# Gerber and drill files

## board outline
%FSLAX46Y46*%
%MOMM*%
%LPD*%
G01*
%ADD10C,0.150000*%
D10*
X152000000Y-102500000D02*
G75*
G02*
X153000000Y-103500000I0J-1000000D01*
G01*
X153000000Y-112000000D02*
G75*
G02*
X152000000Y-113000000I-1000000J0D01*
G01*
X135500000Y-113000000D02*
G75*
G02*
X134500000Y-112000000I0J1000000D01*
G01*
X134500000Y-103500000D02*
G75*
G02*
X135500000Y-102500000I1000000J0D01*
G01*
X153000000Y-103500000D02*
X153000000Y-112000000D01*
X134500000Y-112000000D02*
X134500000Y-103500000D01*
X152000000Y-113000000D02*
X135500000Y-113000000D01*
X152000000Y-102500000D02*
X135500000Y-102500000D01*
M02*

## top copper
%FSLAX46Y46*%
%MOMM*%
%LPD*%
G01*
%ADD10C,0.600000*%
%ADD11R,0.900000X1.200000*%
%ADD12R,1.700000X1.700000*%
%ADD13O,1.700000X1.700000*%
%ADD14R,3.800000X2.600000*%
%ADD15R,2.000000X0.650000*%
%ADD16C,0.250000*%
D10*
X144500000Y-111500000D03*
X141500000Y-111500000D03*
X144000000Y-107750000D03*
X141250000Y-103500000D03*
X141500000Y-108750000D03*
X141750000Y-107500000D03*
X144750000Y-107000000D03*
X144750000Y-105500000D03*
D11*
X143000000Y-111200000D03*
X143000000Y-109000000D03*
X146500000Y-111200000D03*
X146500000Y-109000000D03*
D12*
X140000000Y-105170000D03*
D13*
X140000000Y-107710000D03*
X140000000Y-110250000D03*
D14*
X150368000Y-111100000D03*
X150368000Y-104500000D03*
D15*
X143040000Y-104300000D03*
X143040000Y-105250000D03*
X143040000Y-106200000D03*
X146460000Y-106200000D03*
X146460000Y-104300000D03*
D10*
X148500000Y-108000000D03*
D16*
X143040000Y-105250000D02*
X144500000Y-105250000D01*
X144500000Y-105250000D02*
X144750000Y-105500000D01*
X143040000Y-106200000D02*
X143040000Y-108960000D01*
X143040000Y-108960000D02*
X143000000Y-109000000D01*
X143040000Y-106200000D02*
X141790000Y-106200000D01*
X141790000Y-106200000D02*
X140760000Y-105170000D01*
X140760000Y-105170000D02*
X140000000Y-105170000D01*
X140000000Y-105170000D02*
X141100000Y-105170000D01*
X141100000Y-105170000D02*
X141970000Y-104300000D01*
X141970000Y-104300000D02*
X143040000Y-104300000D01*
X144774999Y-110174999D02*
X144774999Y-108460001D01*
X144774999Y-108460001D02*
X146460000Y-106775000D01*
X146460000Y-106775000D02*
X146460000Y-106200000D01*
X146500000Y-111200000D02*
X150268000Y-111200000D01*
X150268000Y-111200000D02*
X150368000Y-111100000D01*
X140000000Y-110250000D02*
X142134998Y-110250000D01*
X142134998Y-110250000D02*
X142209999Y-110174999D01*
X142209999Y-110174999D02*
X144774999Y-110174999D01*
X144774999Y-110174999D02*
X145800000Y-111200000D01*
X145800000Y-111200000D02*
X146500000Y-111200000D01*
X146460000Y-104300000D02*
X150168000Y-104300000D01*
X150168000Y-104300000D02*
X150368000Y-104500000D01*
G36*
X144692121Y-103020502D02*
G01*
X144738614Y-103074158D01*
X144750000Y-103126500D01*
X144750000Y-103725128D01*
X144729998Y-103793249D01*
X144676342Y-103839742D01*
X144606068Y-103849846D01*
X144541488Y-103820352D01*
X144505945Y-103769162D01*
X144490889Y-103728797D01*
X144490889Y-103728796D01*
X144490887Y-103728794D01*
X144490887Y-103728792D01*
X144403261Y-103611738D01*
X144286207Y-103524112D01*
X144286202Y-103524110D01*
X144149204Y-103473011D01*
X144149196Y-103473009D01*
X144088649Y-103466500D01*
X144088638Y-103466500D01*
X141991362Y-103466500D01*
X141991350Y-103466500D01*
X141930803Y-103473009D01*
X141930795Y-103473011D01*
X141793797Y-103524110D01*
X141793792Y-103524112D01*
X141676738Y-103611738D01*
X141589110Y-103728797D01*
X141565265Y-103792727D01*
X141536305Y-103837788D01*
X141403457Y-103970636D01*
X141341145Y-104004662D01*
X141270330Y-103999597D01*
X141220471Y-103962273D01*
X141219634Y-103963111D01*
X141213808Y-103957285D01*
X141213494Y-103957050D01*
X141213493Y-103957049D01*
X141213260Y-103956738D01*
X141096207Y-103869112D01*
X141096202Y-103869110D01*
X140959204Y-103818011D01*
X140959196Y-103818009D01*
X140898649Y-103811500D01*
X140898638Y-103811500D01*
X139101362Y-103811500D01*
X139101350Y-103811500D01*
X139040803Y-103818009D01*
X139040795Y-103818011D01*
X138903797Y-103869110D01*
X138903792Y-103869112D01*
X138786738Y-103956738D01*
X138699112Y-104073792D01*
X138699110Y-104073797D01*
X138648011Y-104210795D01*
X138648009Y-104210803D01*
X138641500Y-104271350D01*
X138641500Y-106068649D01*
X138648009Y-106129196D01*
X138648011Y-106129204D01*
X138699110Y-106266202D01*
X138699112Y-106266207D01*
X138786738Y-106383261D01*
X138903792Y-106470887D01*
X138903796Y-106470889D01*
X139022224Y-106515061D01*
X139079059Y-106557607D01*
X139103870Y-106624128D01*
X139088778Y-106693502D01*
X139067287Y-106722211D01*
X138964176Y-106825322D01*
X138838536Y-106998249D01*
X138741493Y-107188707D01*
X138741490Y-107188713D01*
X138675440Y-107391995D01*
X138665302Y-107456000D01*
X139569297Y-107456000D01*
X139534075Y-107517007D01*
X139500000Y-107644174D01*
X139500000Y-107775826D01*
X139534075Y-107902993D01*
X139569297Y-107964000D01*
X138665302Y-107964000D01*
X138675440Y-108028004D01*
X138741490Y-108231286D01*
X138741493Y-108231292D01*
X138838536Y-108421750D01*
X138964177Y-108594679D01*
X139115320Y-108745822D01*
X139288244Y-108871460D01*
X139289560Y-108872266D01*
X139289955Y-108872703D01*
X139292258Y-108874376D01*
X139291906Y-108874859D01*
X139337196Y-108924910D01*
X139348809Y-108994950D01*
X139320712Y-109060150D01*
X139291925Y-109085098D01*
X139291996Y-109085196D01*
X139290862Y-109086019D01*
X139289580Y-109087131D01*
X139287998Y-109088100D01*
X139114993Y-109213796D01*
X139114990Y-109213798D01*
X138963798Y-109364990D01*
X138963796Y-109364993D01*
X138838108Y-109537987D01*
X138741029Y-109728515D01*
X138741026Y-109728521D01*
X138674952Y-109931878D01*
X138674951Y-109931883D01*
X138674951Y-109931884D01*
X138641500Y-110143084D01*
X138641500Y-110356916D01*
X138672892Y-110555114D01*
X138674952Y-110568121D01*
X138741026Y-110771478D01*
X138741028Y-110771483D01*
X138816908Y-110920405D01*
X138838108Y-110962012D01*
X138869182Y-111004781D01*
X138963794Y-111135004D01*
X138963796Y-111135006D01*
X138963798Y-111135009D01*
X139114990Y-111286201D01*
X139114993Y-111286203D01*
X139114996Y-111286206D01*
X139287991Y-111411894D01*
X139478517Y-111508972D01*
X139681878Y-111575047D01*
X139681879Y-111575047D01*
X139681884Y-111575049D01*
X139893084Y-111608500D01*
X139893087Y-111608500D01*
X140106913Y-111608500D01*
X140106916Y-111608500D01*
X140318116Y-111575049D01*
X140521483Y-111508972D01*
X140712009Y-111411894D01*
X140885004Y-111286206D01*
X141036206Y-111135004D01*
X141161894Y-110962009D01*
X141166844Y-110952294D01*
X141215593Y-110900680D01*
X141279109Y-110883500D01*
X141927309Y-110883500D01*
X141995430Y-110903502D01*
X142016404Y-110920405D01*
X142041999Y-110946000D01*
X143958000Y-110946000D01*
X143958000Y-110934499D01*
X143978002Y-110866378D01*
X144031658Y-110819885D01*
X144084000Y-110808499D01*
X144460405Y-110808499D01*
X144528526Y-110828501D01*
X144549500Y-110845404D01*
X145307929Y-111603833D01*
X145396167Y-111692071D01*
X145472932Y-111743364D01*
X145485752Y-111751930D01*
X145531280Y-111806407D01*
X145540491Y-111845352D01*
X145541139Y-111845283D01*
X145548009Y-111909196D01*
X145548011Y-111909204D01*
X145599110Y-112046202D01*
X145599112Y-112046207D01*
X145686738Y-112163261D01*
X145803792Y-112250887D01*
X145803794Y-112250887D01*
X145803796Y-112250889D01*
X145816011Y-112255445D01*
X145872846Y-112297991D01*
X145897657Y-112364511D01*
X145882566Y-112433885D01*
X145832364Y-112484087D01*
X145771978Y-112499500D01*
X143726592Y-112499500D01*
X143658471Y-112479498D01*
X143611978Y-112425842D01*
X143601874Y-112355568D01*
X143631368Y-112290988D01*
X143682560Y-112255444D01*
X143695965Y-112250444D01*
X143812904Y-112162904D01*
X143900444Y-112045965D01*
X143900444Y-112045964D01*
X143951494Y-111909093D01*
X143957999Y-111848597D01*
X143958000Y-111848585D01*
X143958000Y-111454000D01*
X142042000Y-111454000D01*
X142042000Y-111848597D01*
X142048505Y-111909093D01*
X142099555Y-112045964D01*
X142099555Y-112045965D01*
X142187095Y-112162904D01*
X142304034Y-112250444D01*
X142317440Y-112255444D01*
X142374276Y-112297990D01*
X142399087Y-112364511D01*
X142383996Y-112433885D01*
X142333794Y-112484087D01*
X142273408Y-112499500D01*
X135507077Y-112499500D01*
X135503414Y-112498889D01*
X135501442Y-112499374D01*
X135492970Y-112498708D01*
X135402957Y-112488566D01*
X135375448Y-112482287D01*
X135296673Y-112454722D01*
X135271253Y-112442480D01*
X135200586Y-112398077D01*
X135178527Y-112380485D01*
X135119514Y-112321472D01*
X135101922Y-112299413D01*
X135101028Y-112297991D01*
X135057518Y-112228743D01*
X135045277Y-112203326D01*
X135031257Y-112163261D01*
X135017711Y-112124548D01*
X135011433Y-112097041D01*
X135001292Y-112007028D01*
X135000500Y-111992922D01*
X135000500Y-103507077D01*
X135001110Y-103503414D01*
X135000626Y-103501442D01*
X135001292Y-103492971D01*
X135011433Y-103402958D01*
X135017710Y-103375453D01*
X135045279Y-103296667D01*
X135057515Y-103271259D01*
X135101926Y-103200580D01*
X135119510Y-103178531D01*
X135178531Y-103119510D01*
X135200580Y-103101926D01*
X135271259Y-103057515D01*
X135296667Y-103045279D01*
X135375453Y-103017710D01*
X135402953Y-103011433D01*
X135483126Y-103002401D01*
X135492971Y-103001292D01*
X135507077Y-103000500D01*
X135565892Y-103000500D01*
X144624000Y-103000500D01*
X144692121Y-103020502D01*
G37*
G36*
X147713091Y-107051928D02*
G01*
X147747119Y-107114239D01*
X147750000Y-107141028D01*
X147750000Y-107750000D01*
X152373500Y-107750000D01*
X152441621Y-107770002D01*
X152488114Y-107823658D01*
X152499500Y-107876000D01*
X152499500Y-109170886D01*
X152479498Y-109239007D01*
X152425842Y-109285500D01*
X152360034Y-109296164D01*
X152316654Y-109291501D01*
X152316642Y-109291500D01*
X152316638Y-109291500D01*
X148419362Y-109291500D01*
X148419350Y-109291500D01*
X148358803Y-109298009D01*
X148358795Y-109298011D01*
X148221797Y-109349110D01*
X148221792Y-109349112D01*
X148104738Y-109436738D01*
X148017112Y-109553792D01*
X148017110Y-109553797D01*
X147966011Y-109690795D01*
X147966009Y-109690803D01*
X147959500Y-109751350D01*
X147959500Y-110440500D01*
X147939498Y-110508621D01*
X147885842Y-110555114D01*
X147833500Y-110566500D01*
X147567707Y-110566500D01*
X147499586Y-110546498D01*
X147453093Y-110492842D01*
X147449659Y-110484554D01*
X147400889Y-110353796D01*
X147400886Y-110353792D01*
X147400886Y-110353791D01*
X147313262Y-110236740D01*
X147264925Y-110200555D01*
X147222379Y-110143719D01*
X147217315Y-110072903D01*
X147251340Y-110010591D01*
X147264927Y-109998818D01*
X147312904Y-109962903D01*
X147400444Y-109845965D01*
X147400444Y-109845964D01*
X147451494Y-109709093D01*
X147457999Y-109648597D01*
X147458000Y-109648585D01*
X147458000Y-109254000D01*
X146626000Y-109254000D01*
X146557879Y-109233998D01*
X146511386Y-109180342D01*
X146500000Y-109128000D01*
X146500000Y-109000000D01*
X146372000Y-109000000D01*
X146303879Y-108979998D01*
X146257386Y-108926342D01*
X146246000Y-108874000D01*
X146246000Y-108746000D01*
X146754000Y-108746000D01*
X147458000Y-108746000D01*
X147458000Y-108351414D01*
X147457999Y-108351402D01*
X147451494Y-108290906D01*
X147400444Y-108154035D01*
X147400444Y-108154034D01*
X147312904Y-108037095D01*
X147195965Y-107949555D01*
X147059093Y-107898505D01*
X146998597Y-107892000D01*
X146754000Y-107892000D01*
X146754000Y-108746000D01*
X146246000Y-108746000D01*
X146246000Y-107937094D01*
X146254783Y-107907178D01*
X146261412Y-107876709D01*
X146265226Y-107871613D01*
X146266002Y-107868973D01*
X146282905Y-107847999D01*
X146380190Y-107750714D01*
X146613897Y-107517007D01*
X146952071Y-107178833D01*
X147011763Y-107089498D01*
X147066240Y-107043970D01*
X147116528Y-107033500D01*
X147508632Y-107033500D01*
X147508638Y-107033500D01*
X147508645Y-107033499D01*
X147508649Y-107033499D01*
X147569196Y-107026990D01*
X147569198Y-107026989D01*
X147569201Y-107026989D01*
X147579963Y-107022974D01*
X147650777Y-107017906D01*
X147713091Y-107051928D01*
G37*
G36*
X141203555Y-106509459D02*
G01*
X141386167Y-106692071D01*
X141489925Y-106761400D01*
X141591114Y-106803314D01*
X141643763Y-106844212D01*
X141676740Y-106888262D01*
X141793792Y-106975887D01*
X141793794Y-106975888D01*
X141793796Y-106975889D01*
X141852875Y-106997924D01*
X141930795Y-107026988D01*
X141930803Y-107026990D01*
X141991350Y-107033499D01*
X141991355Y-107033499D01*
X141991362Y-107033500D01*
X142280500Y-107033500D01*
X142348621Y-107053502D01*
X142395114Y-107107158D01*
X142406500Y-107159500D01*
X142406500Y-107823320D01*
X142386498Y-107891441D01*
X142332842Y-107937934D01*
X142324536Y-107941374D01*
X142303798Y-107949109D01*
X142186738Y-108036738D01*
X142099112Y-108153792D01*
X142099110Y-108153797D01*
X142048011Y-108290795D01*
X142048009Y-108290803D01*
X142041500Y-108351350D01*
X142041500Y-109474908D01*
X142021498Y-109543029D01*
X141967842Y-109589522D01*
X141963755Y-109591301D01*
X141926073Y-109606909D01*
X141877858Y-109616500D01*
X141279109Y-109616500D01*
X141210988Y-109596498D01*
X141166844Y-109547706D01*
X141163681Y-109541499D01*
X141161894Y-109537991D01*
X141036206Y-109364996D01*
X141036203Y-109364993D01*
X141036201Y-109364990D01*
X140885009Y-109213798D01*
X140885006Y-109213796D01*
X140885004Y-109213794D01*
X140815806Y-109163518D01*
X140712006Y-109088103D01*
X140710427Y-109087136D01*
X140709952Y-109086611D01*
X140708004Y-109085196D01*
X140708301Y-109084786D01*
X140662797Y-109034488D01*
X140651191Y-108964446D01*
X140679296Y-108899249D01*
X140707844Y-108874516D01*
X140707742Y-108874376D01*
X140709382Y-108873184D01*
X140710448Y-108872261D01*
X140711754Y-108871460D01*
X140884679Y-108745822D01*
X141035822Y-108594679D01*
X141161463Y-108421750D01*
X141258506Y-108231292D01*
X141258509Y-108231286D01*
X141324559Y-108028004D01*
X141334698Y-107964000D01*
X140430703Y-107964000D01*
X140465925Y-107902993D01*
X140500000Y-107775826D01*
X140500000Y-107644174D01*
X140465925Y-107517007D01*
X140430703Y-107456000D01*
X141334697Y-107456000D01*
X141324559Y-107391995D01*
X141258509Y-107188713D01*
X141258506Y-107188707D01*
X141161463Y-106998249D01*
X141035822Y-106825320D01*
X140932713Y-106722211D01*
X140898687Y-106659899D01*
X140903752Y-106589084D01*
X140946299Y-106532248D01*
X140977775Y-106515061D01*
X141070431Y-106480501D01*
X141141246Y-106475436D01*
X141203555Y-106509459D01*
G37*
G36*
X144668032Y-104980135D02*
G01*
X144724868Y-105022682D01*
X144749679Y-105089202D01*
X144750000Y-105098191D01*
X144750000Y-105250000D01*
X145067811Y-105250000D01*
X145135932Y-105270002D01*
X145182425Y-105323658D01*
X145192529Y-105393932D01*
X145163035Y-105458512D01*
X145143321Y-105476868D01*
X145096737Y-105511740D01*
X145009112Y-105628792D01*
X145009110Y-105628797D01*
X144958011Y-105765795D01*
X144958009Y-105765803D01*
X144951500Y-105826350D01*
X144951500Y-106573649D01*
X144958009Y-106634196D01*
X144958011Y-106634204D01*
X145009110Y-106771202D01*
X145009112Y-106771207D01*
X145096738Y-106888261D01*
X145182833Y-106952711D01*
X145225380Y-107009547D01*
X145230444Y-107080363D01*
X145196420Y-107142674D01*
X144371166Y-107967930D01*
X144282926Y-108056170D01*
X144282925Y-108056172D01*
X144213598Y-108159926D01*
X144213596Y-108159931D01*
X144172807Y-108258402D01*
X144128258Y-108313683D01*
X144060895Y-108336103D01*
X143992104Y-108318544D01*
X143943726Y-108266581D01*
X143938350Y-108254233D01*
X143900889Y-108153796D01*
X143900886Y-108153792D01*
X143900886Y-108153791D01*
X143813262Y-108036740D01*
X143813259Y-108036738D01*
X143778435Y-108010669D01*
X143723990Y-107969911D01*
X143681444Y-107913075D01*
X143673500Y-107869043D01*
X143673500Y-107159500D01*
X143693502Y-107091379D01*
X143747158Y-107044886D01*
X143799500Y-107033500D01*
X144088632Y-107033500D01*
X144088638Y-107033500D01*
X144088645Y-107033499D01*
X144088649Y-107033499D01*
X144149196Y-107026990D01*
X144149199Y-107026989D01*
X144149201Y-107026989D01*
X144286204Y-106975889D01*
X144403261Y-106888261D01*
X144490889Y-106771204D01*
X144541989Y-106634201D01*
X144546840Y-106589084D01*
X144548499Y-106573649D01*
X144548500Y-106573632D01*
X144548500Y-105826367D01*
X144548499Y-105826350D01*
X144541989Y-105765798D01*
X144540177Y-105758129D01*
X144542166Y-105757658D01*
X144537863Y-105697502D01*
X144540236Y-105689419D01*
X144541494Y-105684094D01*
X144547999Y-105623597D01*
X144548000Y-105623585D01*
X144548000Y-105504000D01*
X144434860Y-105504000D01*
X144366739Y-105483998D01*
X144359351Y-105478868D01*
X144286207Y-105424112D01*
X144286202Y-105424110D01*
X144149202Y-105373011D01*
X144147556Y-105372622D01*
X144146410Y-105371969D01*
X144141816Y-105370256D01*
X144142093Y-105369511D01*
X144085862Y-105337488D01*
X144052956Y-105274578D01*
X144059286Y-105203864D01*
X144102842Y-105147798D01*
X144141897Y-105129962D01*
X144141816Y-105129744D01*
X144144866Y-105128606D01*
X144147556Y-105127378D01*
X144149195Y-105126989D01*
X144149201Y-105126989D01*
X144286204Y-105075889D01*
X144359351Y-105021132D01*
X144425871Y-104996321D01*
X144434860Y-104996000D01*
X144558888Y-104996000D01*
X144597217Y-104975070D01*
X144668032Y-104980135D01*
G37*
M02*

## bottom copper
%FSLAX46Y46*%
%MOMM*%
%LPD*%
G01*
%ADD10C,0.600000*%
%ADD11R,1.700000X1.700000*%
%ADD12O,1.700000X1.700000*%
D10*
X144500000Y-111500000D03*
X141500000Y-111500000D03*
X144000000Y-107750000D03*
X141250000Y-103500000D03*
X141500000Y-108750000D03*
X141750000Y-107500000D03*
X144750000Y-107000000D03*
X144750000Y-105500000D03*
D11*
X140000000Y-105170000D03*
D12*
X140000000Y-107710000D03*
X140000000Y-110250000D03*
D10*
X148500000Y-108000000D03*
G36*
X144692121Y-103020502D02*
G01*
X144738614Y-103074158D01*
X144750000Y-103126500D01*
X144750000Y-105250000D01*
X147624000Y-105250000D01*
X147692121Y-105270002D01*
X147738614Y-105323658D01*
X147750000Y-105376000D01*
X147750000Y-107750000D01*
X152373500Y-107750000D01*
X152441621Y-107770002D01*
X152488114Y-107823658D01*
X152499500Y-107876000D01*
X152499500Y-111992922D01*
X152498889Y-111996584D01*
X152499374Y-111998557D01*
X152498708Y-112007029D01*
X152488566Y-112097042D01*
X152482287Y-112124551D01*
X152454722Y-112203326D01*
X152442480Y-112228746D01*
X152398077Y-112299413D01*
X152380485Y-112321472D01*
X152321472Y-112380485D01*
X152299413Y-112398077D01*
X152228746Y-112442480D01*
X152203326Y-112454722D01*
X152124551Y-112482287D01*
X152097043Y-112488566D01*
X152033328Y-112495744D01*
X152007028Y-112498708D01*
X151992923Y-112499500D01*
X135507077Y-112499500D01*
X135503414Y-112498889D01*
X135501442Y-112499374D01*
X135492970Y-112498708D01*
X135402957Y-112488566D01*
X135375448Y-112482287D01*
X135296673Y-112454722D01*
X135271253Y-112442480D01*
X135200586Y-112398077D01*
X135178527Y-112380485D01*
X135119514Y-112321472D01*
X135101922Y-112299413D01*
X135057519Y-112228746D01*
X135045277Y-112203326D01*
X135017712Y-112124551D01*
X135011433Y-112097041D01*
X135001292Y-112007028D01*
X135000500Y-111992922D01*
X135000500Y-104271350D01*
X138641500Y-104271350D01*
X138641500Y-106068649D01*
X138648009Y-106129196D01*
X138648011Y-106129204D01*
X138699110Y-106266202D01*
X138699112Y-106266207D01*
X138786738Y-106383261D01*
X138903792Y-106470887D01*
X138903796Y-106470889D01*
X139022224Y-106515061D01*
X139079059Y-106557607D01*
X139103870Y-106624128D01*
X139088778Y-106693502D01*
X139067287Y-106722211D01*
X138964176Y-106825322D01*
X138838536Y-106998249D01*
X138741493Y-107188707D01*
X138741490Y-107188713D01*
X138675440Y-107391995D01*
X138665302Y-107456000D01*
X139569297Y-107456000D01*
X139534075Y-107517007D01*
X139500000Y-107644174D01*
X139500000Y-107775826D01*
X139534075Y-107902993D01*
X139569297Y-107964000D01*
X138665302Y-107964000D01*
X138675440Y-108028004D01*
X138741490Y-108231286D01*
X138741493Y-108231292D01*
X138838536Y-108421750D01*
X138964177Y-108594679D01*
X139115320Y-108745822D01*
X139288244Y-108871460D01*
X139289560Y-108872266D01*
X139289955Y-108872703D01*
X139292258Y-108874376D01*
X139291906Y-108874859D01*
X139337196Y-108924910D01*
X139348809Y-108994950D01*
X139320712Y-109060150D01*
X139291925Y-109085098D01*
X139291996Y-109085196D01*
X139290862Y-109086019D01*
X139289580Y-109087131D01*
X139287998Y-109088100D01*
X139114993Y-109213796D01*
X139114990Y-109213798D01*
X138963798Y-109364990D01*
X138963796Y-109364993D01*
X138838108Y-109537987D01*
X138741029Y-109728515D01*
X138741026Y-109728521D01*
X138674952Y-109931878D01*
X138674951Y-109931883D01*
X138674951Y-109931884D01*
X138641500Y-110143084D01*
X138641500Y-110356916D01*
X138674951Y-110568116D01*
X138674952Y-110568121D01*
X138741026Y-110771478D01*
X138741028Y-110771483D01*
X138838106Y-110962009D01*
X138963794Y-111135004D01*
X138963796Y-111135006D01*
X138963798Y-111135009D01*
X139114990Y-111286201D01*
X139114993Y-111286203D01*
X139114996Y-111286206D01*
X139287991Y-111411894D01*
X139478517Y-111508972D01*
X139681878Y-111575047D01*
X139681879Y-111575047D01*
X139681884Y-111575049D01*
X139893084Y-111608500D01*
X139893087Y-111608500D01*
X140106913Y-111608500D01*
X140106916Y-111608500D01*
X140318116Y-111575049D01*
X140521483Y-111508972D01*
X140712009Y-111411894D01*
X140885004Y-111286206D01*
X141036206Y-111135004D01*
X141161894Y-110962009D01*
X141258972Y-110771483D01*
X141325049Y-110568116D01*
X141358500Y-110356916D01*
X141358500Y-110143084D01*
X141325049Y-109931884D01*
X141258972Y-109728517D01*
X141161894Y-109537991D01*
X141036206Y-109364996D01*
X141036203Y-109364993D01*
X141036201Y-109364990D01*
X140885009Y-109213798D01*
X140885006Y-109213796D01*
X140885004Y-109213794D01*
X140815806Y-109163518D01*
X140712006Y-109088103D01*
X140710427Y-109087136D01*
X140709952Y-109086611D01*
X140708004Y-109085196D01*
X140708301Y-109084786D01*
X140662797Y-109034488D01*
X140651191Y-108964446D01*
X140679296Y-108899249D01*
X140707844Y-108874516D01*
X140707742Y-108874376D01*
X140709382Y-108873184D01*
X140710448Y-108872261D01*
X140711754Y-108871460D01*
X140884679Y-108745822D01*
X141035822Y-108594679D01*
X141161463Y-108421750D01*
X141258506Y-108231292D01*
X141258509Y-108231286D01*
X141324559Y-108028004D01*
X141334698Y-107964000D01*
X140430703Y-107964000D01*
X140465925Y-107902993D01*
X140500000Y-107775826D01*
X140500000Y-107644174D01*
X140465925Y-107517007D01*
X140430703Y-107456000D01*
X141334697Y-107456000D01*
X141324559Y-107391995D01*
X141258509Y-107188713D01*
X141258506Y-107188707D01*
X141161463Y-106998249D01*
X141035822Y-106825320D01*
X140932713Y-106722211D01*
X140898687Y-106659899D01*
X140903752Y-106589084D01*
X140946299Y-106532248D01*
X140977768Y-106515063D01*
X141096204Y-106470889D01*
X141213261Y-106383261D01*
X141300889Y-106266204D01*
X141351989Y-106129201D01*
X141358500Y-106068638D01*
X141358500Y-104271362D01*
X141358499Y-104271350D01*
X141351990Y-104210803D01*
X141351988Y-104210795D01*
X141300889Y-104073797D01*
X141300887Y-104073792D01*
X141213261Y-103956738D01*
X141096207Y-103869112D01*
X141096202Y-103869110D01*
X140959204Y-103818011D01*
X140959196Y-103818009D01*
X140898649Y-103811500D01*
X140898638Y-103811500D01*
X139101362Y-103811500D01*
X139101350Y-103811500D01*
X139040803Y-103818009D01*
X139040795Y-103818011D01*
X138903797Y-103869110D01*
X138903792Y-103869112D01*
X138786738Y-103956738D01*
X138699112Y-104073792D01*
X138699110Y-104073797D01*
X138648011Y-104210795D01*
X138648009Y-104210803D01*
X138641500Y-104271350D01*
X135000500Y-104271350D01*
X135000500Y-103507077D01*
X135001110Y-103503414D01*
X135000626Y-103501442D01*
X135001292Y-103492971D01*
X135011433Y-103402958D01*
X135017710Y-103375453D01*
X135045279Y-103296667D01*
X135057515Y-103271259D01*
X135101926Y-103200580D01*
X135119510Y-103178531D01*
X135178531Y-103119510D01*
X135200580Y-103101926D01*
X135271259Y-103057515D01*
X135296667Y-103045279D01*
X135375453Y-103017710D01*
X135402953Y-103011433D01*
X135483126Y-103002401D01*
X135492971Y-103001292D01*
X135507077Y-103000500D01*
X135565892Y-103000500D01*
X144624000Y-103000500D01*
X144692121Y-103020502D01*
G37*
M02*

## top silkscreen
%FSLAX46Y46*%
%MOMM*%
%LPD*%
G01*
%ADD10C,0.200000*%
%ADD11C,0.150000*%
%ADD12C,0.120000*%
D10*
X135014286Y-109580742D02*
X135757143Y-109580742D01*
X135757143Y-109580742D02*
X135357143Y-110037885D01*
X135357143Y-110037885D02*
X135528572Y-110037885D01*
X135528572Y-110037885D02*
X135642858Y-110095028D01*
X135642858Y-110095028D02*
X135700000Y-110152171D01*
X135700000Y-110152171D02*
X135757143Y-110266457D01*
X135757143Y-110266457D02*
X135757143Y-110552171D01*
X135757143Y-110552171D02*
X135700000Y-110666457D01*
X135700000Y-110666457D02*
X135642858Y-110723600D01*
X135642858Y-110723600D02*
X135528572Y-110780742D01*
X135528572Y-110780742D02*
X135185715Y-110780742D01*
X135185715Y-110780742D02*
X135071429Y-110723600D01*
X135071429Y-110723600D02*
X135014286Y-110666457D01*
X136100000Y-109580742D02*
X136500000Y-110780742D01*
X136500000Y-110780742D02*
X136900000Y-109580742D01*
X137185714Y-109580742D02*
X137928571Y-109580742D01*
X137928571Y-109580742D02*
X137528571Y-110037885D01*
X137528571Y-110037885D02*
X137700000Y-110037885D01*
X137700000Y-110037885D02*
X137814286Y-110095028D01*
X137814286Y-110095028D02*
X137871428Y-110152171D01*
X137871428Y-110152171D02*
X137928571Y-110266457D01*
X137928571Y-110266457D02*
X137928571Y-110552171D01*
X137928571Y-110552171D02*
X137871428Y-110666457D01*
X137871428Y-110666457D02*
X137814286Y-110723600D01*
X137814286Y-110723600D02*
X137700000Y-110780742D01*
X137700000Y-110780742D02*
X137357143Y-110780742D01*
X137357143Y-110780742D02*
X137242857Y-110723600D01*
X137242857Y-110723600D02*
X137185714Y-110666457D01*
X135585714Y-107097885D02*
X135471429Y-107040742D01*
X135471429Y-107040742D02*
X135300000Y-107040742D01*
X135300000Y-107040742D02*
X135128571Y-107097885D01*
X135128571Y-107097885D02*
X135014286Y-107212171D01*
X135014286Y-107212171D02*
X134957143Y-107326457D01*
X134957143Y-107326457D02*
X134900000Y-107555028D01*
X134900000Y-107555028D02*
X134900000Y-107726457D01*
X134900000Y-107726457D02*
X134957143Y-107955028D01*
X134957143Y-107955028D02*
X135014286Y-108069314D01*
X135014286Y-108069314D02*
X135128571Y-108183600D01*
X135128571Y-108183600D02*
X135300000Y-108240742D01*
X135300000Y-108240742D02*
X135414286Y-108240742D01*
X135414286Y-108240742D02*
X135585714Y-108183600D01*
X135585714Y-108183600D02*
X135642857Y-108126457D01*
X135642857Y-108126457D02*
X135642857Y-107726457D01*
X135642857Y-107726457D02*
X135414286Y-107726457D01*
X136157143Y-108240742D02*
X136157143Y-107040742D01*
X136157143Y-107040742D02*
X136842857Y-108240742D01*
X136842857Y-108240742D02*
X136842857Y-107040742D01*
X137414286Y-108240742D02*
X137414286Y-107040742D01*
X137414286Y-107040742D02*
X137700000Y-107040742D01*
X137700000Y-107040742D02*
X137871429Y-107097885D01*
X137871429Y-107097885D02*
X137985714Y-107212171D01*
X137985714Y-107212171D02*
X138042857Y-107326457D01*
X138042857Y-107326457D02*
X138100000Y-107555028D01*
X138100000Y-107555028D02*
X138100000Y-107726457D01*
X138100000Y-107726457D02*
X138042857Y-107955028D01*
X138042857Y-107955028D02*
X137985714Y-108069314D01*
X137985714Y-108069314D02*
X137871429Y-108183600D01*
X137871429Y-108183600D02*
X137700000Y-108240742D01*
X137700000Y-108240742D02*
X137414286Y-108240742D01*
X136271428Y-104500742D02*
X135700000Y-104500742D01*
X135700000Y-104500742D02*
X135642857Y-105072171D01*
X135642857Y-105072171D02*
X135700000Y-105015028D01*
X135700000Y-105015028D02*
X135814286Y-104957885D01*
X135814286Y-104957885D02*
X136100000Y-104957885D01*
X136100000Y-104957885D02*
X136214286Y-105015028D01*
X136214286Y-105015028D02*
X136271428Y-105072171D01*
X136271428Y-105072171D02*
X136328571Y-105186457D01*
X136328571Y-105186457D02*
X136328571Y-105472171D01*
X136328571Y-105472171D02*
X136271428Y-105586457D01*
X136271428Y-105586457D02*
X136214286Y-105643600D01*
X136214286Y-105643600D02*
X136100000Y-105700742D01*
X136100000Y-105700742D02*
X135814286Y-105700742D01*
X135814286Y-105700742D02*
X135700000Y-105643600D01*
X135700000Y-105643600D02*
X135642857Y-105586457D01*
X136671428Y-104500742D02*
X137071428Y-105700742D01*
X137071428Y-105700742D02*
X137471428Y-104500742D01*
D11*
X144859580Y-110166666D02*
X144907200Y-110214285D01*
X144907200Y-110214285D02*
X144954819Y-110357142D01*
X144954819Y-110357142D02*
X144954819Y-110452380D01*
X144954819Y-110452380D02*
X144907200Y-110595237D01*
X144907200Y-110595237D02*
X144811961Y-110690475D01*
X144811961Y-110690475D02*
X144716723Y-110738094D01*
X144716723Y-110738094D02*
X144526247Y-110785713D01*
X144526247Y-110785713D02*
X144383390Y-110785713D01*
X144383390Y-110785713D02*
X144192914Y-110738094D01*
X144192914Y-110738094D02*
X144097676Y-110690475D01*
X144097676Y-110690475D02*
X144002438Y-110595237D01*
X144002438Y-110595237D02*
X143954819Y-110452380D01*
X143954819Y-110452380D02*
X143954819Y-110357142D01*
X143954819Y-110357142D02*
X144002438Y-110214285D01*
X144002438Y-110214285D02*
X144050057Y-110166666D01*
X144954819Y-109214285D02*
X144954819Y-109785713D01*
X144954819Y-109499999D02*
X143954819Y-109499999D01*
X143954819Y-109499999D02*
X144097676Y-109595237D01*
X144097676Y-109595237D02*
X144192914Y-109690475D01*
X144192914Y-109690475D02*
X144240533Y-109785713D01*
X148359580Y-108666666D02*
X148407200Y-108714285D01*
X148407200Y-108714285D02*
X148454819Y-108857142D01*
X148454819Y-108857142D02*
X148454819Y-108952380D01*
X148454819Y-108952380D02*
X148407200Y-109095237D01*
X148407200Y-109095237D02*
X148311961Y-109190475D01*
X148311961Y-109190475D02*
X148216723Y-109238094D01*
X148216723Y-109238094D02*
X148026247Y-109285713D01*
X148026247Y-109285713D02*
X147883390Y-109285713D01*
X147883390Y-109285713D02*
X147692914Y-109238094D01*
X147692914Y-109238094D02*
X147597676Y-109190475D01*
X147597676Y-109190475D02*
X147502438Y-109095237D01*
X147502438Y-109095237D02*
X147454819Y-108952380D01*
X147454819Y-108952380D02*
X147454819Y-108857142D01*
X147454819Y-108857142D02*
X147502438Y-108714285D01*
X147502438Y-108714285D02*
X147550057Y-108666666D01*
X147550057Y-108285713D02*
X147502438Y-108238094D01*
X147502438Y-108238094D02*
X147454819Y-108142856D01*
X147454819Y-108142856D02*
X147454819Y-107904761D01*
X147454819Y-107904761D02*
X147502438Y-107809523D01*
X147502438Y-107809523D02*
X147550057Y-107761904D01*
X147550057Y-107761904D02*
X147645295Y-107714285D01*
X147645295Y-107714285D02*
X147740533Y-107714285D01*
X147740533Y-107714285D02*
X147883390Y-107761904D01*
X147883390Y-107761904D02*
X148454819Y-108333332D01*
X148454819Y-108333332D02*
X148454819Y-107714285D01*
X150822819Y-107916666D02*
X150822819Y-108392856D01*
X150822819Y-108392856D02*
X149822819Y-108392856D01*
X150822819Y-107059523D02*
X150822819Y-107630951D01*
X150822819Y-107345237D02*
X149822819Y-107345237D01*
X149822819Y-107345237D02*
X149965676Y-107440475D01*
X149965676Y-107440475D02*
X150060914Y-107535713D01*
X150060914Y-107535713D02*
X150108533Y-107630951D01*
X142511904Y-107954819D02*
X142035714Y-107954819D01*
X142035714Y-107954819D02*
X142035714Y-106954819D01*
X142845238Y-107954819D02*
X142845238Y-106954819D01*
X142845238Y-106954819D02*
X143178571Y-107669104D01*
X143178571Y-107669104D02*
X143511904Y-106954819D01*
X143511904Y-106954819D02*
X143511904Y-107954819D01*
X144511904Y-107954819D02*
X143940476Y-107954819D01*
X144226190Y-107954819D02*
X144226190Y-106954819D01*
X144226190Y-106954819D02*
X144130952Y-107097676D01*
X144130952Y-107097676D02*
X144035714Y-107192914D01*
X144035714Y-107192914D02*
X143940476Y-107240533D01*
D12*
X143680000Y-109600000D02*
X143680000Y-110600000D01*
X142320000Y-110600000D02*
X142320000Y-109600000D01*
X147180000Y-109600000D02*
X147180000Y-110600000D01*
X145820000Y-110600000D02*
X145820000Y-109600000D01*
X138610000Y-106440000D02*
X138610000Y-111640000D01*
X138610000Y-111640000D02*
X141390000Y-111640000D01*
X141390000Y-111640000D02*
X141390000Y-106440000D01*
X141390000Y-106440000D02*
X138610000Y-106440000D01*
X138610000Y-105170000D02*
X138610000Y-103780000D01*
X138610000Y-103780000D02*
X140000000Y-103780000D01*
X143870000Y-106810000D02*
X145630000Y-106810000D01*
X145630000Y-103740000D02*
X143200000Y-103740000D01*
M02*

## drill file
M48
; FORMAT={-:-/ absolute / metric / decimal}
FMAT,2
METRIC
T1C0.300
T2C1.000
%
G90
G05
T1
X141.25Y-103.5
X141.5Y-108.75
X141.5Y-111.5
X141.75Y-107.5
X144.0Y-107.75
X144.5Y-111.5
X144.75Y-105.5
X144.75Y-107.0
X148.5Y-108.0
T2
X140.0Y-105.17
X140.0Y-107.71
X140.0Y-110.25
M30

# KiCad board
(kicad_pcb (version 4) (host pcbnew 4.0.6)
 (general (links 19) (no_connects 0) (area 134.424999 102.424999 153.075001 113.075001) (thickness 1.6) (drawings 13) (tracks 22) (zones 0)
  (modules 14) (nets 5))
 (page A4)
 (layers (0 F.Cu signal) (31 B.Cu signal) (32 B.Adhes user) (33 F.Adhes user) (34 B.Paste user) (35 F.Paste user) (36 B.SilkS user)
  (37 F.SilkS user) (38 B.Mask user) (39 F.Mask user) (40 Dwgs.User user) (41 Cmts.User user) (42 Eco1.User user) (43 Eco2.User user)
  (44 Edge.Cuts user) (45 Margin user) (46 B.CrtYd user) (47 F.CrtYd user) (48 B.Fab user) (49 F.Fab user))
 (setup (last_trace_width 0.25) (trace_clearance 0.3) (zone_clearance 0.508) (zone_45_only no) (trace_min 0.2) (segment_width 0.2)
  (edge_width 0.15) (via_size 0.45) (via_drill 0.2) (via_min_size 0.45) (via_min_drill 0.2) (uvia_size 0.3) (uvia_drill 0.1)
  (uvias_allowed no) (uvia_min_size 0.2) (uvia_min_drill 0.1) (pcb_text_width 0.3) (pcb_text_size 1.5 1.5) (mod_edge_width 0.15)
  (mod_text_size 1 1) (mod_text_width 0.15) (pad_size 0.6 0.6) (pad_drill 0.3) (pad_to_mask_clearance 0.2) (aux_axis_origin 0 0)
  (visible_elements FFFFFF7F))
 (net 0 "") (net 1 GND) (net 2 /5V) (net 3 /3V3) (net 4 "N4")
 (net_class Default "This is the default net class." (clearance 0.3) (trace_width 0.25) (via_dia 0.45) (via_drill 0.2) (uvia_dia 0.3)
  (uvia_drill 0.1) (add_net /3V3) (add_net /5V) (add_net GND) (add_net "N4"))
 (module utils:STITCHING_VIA (layer F.Cu) (at 144.5 111.5)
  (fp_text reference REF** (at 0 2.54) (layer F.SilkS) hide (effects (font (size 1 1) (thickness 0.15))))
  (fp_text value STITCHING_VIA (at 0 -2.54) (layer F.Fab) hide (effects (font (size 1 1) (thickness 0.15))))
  (pad 1 thru_hole circle (at 0 0) (size 0.6 0.6) (drill 0.3) (layers *.Cu) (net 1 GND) (zone_connect 2)))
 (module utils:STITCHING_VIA (layer F.Cu) (at 141.5 111.5)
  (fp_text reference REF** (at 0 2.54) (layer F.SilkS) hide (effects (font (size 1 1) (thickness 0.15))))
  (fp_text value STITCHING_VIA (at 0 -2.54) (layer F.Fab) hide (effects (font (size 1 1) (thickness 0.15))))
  (pad 1 thru_hole circle (at 0 0) (size 0.6 0.6) (drill 0.3) (layers *.Cu) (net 1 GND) (zone_connect 2)))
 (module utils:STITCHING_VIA (layer F.Cu) (at 144 107.75)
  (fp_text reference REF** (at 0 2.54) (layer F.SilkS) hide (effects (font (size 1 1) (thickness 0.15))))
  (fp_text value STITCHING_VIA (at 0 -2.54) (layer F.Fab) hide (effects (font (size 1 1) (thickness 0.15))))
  (pad 1 thru_hole circle (at 0 0) (size 0.6 0.6) (drill 0.3) (layers *.Cu) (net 1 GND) (zone_connect 2)))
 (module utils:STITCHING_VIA (layer F.Cu) (at 141.25 103.5)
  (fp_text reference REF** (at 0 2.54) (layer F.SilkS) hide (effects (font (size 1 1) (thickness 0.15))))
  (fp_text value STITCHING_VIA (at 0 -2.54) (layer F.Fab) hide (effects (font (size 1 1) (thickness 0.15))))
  (pad 1 thru_hole circle (at 0 0) (size 0.6 0.6) (drill 0.3) (layers *.Cu) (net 1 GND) (zone_connect 2)))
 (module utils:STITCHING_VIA (layer F.Cu) (at 141.5 108.75)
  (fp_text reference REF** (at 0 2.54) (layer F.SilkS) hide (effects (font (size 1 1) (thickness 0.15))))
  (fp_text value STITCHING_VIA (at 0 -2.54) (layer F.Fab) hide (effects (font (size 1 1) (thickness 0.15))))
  (pad 1 thru_hole circle (at 0 0) (size 0.6 0.6) (drill 0.3) (layers *.Cu) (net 1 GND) (zone_connect 2)))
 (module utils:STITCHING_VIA (layer F.Cu) (at 141.75 107.5)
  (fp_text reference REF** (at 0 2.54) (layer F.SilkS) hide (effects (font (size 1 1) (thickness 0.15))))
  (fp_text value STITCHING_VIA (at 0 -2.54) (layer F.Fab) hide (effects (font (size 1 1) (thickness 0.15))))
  (pad 1 thru_hole circle (at 0 0) (size 0.6 0.6) (drill 0.3) (layers *.Cu) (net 1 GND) (zone_connect 2)))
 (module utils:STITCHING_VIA (layer F.Cu) (at 144.75 107)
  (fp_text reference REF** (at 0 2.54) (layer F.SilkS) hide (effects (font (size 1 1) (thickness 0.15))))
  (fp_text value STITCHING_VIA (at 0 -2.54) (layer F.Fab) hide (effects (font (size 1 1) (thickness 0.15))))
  (pad 1 thru_hole circle (at 0 0) (size 0.6 0.6) (drill 0.3) (layers *.Cu) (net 1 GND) (zone_connect 2)))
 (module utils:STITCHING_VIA (layer F.Cu) (at 144.75 105.5)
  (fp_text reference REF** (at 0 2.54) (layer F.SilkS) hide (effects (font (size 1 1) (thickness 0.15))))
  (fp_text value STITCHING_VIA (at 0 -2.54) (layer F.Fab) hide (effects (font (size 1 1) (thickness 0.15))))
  (pad 1 thru_hole circle (at 0 0) (size 0.6 0.6) (drill 0.3) (layers *.Cu) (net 1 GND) (zone_connect 2)))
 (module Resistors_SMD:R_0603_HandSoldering (layer F.Cu) (at 143 110.1 90)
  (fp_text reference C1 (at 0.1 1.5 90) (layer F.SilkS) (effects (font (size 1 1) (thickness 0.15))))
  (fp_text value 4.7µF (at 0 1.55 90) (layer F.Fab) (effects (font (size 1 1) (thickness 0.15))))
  (fp_line (start 0.5 0.68) (end -0.5 0.68) (layer F.SilkS) (width 0.12))
  (fp_line (start -0.5 -0.68) (end 0.5 -0.68) (layer F.SilkS) (width 0.12))
  (pad 1 smd rect (at -1.1 0 90) (size 1.2 0.9) (layers F.Cu F.Paste F.Mask) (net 1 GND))
  (pad 2 smd rect (at 1.1 0 90) (size 1.2 0.9) (layers F.Cu F.Paste F.Mask) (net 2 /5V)))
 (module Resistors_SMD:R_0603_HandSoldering (layer F.Cu) (at 146.5 110.1 90)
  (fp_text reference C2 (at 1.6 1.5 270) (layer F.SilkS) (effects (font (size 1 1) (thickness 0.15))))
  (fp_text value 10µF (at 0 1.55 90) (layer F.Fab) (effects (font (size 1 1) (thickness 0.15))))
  (fp_line (start 0.5 0.68) (end -0.5 0.68) (layer F.SilkS) (width 0.12))
  (fp_line (start -0.5 -0.68) (end 0.5 -0.68) (layer F.SilkS) (width 0.12))
  (pad 1 smd rect (at -1.1 0 90) (size 1.2 0.9) (layers F.Cu F.Paste F.Mask) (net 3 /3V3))
  (pad 2 smd rect (at 1.1 0 90) (size 1.2 0.9) (layers F.Cu F.Paste F.Mask) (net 1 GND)))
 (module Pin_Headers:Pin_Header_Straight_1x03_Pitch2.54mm (layer F.Cu) (at 140 105.17)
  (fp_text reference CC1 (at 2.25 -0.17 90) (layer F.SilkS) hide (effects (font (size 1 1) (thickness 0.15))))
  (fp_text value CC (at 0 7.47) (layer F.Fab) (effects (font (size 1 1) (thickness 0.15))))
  (fp_line (start -1.39 1.27) (end -1.39 6.47) (layer F.SilkS) (width 0.12))
  (fp_line (start -1.39 6.47) (end 1.39 6.47) (layer F.SilkS) (width 0.12))
  (fp_line (start 1.39 6.47) (end 1.39 1.27) (layer F.SilkS) (width 0.12))
  (fp_line (start 1.39 1.27) (end -1.39 1.27) (layer F.SilkS) (width 0.12))
  (fp_line (start -1.39 0) (end -1.39 -1.39) (layer F.SilkS) (width 0.12))
  (fp_line (start -1.39 -1.39) (end 0 -1.39) (layer F.SilkS) (width 0.12))
  (pad 1 thru_hole rect (at 0 0) (size 1.7 1.7) (drill 1) (layers *.Cu *.Mask) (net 2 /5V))
  (pad 2 thru_hole oval (at 0 2.54) (size 1.7 1.7) (drill 1) (layers *.Cu *.Mask) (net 1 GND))
  (pad 3 thru_hole oval (at 0 5.08) (size 1.7 1.7) (drill 1) (layers *.Cu *.Mask) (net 3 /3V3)))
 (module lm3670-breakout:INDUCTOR (layer F.Cu) (at 150.368 107.8 90)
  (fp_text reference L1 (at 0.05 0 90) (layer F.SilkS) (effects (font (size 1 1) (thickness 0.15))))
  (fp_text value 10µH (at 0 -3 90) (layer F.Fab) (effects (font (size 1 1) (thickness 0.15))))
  (pad 1 smd rect (at -3.3 0 90) (size 2.6 3.8) (layers F.Cu F.Paste F.Mask) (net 3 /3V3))
  (pad 2 smd rect (at 3.3 0 90) (size 2.6 3.8) (layers F.Cu F.Paste F.Mask) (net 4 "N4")))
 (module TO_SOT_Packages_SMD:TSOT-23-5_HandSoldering (layer F.Cu) (at 144.75 105.25)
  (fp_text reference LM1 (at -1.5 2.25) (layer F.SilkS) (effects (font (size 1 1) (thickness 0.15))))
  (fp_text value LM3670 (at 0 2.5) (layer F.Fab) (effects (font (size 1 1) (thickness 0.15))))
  (fp_line (start -0.88 1.56) (end 0.88 1.56) (layer F.SilkS) (width 0.12))
  (fp_line (start 0.88 -1.51) (end -1.55 -1.51) (layer F.SilkS) (width 0.12))
  (pad 1 smd rect (at -1.71 -0.95) (size 2 0.65) (layers F.Cu F.Paste F.Mask) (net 2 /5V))
  (pad 2 smd rect (at -1.71 0) (size 2 0.65) (layers F.Cu F.Paste F.Mask) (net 1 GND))
  (pad 3 smd rect (at -1.71 0.95) (size 2 0.65) (layers F.Cu F.Paste F.Mask) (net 2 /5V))
  (pad 4 smd rect (at 1.71 0.95) (size 2 0.65) (layers F.Cu F.Paste F.Mask) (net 3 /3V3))
  (pad 5 smd rect (at 1.71 -0.95) (size 2 0.65) (layers F.Cu F.Paste F.Mask) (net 4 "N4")))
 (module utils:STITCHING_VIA (layer F.Cu) (at 148.5 108)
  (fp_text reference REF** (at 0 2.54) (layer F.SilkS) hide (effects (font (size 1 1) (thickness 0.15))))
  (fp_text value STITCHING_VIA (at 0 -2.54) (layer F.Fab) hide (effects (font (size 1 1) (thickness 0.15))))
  (pad 1 thru_hole circle (at 0 0) (size 0.6 0.6) (drill 0.3) (layers *.Cu) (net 1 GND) (zone_connect 2)))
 (gr_arc (start 152 103.5) (end 152 102.5) (angle 90) (layer Edge.Cuts) (width 0.15))
 (gr_arc (start 152 112) (end 153 112) (angle 90) (layer Edge.Cuts) (width 0.15))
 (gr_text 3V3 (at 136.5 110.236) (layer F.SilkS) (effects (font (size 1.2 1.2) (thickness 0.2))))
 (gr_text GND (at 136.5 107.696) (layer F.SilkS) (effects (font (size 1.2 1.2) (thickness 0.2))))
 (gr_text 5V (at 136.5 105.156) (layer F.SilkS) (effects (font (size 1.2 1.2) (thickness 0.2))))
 (gr_arc (start 135.5 112) (end 135.5 113) (angle 90) (layer Edge.Cuts) (width 0.15))
 (gr_arc (start 135.5 103.5) (end 134.5 103.5) (angle 90) (layer Edge.Cuts) (width 0.15))
 (gr_line (start 153 103.5) (end 153 112) (layer Edge.Cuts) (width 0.15))
 (gr_line (start 134.5 112) (end 134.5 103.5) (layer Edge.Cuts) (width 0.15))
 (gr_line (start 152 113) (end 135.5 113) (layer Edge.Cuts) (width 0.15))
 (gr_line (start 152 102.5) (end 135.5 102.5) (layer Edge.Cuts) (width 0.15))
 (segment (start 143.04 105.25) (end 144.5 105.25) (width 0.25) (layer F.Cu) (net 1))
 (segment (start 144.5 105.25) (end 144.75 105.5) (width 0.25) (layer F.Cu) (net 1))
 (segment (start 143.04 106.2) (end 143.04 108.96) (width 0.25) (layer F.Cu) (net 2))
 (segment (start 143.04 108.96) (end 143 109) (width 0.25) (layer F.Cu) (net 2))
 (segment (start 143.04 106.2) (end 141.79 106.2) (width 0.25) (layer F.Cu) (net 2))
 (segment (start 141.79 106.2) (end 140.76 105.17) (width 0.25) (layer F.Cu) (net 2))
 (segment (start 140.76 105.17) (end 140 105.17) (width 0.25) (layer F.Cu) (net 2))
 (segment (start 140 105.17) (end 141.1 105.17) (width 0.25) (layer F.Cu) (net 2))
 (segment (start 141.1 105.17) (end 141.97 104.3) (width 0.25) (layer F.Cu) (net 2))
 (segment (start 141.97 104.3) (end 143.04 104.3) (width 0.25) (layer F.Cu) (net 2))
 (segment (start 144.774999 110.174999) (end 144.774999 108.460001) (width 0.25) (layer F.Cu) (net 3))
 (segment (start 144.774999 108.460001) (end 146.46 106.775) (width 0.25) (layer F.Cu) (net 3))
 (segment (start 146.46 106.775) (end 146.46 106.2) (width 0.25) (layer F.Cu) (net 3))
 (segment (start 146.5 111.2) (end 150.268 111.2) (width 0.25) (layer F.Cu) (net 3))
 (segment (start 150.268 111.2) (end 150.368 111.1) (width 0.25) (layer F.Cu) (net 3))
 (segment (start 140 110.25) (end 142.134998 110.25) (width 0.25) (layer F.Cu) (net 3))
 (segment (start 142.134998 110.25) (end 142.209999 110.174999) (width 0.25) (layer F.Cu) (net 3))
 (segment (start 142.209999 110.174999) (end 144.774999 110.174999) (width 0.25) (layer F.Cu) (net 3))
 (segment (start 144.774999 110.174999) (end 145.8 111.2) (width 0.25) (layer F.Cu) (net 3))
 (segment (start 145.8 111.2) (end 146.5 111.2) (width 0.25) (layer F.Cu) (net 3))
 (segment (start 146.46 104.3) (end 150.168 104.3) (width 0.25) (layer F.Cu) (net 4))
 (segment (start 150.168 104.3) (end 150.368 104.5) (width 0.25) (layer F.Cu) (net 4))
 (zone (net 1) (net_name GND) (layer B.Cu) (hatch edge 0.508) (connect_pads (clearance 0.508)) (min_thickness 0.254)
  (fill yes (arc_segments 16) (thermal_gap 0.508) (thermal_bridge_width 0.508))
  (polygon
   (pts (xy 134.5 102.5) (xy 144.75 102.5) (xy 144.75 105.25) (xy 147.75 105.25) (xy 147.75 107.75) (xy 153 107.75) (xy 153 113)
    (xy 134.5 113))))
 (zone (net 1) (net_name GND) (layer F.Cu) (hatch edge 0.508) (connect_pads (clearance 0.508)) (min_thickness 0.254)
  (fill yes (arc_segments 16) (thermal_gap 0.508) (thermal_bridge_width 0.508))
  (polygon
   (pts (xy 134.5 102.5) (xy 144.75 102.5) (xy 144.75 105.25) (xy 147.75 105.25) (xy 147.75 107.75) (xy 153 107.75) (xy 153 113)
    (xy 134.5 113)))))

